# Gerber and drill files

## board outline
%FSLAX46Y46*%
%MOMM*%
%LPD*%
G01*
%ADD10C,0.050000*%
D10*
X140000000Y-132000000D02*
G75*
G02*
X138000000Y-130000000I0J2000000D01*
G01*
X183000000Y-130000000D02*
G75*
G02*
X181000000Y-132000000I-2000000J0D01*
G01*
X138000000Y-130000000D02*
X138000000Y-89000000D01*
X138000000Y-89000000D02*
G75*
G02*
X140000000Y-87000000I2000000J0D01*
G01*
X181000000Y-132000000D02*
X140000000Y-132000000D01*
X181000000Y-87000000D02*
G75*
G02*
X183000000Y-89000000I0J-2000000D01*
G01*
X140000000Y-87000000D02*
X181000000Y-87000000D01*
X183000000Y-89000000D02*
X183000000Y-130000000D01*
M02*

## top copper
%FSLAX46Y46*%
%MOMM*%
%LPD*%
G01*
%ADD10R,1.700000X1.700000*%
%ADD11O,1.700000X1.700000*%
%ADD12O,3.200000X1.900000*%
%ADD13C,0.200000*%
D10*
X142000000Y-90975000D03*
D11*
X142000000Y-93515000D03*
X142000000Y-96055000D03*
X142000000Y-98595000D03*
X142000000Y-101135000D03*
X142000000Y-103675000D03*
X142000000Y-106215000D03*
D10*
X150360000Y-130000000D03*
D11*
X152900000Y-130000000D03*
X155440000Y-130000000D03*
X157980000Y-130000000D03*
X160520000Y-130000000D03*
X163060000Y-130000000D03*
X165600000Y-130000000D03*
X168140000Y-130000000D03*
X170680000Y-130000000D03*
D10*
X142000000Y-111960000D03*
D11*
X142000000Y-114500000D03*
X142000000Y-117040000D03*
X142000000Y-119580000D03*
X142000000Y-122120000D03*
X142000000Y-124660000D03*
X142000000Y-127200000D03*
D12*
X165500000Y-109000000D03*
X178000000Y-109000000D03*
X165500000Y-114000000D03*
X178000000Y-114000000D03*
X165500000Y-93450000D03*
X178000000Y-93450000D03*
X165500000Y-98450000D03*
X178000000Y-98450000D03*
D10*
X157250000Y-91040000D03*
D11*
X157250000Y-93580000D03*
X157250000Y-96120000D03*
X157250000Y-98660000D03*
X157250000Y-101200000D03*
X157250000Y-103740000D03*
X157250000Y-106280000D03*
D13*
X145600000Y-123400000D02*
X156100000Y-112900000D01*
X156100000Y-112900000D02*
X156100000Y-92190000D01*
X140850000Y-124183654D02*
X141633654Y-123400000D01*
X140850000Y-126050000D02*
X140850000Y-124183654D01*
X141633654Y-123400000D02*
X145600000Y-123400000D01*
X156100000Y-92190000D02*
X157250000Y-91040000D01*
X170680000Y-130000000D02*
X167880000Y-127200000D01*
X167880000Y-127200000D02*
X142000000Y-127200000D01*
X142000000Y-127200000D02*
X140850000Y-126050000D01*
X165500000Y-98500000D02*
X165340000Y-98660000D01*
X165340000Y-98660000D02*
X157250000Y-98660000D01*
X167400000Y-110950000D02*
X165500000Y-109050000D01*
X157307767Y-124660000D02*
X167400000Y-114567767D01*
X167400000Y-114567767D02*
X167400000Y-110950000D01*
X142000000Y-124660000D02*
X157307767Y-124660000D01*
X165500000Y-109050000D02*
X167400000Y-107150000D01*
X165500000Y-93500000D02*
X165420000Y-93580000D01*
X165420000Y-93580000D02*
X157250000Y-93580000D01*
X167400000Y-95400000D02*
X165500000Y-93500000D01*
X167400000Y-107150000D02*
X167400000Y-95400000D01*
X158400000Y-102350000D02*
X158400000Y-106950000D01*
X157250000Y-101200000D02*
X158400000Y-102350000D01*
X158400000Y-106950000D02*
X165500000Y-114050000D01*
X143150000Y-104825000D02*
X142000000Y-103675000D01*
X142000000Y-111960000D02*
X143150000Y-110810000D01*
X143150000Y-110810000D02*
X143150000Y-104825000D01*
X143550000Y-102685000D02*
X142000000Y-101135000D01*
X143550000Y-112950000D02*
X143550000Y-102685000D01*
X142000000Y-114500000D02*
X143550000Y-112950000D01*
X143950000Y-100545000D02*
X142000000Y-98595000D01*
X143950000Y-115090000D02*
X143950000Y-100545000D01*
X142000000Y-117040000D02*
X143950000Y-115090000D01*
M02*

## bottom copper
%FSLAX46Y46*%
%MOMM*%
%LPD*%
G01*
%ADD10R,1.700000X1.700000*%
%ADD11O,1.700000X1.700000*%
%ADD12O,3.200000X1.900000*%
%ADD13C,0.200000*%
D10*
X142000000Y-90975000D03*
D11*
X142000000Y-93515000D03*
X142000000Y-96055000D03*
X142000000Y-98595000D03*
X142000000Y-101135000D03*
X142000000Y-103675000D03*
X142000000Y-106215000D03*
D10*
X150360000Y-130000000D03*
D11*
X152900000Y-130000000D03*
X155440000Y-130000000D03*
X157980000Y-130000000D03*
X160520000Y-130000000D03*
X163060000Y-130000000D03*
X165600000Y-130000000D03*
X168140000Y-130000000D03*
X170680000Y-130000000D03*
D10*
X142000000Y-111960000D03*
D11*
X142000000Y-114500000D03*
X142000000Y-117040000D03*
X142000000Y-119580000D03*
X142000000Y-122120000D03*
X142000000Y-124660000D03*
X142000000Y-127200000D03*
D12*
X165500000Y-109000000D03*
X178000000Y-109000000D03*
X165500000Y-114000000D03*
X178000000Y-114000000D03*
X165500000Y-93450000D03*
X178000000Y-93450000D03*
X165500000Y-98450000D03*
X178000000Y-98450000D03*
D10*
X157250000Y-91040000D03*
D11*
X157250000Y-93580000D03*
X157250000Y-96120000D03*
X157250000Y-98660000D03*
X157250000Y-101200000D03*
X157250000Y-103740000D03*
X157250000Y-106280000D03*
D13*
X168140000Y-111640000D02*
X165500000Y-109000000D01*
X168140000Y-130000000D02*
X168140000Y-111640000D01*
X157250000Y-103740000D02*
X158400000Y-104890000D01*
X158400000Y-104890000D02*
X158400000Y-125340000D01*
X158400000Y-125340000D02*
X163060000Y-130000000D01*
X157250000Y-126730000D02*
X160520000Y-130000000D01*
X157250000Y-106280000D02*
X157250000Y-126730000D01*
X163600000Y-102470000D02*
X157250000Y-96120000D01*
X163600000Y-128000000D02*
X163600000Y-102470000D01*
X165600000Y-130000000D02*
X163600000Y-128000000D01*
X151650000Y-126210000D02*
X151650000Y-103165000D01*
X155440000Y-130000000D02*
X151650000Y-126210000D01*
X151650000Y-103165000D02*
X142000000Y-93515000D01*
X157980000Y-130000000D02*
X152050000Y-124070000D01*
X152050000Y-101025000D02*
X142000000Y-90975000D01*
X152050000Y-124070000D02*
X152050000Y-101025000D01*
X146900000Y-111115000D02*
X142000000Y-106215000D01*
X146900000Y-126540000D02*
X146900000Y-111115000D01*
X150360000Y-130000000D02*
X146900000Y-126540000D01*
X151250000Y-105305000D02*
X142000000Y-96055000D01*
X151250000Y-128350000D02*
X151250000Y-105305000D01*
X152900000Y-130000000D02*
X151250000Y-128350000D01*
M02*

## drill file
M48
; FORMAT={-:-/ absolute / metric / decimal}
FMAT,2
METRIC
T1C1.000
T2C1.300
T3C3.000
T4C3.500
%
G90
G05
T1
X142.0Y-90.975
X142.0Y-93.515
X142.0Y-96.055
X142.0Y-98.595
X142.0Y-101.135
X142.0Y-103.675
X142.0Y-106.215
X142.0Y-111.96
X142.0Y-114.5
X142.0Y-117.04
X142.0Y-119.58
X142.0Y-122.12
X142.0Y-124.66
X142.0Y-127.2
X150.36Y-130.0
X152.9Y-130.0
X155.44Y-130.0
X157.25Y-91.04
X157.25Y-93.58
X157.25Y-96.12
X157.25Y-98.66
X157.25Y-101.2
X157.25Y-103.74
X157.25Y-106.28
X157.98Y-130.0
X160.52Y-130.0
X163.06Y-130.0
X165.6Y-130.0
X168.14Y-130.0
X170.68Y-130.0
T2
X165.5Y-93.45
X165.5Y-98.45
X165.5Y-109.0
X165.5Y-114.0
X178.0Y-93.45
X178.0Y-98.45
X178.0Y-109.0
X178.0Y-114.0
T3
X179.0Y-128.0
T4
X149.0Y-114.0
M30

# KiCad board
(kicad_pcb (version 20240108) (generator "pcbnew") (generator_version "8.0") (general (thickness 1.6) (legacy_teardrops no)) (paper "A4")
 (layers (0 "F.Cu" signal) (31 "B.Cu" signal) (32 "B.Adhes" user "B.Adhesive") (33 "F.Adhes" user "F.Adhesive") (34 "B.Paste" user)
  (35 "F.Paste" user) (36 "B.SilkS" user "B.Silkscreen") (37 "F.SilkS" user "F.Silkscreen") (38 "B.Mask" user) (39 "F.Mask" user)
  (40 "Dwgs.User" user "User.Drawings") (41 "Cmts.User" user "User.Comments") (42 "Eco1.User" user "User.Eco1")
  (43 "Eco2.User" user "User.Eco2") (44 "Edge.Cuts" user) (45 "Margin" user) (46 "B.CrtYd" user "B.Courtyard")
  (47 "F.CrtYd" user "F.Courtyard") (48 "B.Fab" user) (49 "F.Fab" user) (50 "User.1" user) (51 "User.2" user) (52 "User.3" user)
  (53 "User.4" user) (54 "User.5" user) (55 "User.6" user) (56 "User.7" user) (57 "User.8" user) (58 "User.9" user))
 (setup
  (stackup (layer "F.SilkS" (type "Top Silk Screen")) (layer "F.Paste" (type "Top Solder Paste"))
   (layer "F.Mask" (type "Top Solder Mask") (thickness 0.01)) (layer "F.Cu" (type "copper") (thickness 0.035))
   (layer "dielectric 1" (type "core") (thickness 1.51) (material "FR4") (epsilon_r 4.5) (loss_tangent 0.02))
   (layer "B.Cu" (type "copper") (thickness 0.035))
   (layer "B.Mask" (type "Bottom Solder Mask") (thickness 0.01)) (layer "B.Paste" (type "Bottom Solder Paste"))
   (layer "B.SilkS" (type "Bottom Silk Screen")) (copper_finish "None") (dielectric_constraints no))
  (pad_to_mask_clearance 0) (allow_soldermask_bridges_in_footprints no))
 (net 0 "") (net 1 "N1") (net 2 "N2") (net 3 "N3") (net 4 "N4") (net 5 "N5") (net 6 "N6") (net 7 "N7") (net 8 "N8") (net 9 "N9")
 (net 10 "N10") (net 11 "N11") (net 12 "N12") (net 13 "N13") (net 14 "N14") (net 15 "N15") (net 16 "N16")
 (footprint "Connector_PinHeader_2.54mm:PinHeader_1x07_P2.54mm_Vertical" (layer "F.Cu") (at 142 90.975)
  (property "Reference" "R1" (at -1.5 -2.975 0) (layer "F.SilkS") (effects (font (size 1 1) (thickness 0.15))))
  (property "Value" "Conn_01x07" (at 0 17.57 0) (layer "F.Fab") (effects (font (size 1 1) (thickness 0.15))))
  (pad "1" thru_hole rect (at 0 0) (size 1.7 1.7) (drill 1) (layers "*.Cu" "*.Mask") (remove_unused_layers no) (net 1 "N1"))
  (pad "2" thru_hole oval (at 0 2.54) (size 1.7 1.7) (drill 1) (layers "*.Cu" "*.Mask") (remove_unused_layers no) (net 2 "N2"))
  (pad "3" thru_hole oval (at 0 5.08) (size 1.7 1.7) (drill 1) (layers "*.Cu" "*.Mask") (remove_unused_layers no) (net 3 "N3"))
  (pad "4" thru_hole oval (at 0 7.62) (size 1.7 1.7) (drill 1) (layers "*.Cu" "*.Mask") (remove_unused_layers no) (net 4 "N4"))
  (pad "5" thru_hole oval (at 0 10.16) (size 1.7 1.7) (drill 1) (layers "*.Cu" "*.Mask") (remove_unused_layers no) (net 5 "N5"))
  (pad "6" thru_hole oval (at 0 12.7) (size 1.7 1.7) (drill 1) (layers "*.Cu" "*.Mask") (remove_unused_layers no) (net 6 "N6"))
  (pad "7" thru_hole oval (at 0 15.24) (size 1.7 1.7) (drill 1) (layers "*.Cu" "*.Mask") (remove_unused_layers no) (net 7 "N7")))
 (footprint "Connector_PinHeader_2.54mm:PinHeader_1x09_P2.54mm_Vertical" (layer "F.Cu") (at 150.36 130 90)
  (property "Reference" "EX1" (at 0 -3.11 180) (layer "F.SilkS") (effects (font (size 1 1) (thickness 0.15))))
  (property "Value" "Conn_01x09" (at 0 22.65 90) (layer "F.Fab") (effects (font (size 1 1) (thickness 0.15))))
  (pad "1" thru_hole rect (at 0 0 90) (size 1.7 1.7) (drill 1) (layers "*.Cu" "*.Mask") (remove_unused_layers no) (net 7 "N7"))
  (pad "2" thru_hole oval (at 0 2.54 90) (size 1.7 1.7) (drill 1) (layers "*.Cu" "*.Mask") (remove_unused_layers no) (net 3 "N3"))
  (pad "3" thru_hole oval (at 0 5.08 90) (size 1.7 1.7) (drill 1) (layers "*.Cu" "*.Mask") (remove_unused_layers no) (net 2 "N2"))
  (pad "4" thru_hole oval (at 0 7.62 90) (size 1.7 1.7) (drill 1) (layers "*.Cu" "*.Mask") (remove_unused_layers no) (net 1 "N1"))
  (pad "5" thru_hole oval (at 0 10.16 90) (size 1.7 1.7) (drill 1) (layers "*.Cu" "*.Mask") (remove_unused_layers no) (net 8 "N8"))
  (pad "6" thru_hole oval (at 0 12.7 90) (size 1.7 1.7) (drill 1) (layers "*.Cu" "*.Mask") (remove_unused_layers no) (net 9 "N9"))
  (pad "7" thru_hole oval (at 0 15.24 90) (size 1.7 1.7) (drill 1) (layers "*.Cu" "*.Mask") (remove_unused_layers no) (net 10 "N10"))
  (pad "8" thru_hole oval (at 0 17.78 90) (size 1.7 1.7) (drill 1) (layers "*.Cu" "*.Mask") (remove_unused_layers no) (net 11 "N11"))
  (pad "9" thru_hole oval (at 0 20.32 90) (size 1.7 1.7) (drill 1) (layers "*.Cu" "*.Mask") (remove_unused_layers no) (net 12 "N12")))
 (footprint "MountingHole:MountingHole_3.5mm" (layer "F.Cu") (at 149 114)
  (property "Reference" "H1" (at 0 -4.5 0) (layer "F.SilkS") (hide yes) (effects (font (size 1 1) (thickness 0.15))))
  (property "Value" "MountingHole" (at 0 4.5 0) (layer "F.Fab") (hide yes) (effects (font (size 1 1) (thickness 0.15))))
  (pad "" np_thru_hole circle (at 0 0) (size 3.5 3.5) (drill 3.5) (layers "*.Cu" "*.Mask")))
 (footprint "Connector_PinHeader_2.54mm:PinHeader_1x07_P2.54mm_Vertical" (layer "F.Cu") (at 142 111.96)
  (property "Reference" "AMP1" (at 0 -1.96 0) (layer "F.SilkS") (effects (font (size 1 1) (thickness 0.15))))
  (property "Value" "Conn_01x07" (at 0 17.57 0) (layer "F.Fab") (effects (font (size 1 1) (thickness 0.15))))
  (pad "1" thru_hole rect (at 0 0) (size 1.7 1.7) (drill 1) (layers "*.Cu" "*.Mask") (remove_unused_layers no) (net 6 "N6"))
  (pad "2" thru_hole oval (at 0 2.54) (size 1.7 1.7) (drill 1) (layers "*.Cu" "*.Mask") (remove_unused_layers no) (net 5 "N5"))
  (pad "3" thru_hole oval (at 0 5.08) (size 1.7 1.7) (drill 1) (layers "*.Cu" "*.Mask") (remove_unused_layers no) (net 4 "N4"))
  (pad "4" thru_hole oval (at 0 7.62) (size 1.7 1.7) (drill 1) (layers "*.Cu" "*.Mask") (remove_unused_layers no) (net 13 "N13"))
  (pad "5" thru_hole oval (at 0 10.16) (size 1.7 1.7) (drill 1) (layers "*.Cu" "*.Mask") (remove_unused_layers no) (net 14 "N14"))
  (pad "6" thru_hole oval (at 0 12.7) (size 1.7 1.7) (drill 1) (layers "*.Cu" "*.Mask") (remove_unused_layers no) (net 11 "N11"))
  (pad "7" thru_hole oval (at 0 15.24) (size 1.7 1.7) (drill 1) (layers "*.Cu" "*.Mask") (remove_unused_layers no) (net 12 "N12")))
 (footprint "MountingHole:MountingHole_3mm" (layer "F.Cu") (at 179 128)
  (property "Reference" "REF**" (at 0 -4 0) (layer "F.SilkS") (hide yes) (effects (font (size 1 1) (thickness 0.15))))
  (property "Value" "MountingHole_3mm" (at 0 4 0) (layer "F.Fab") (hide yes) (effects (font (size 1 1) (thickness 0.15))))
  (pad "" np_thru_hole circle (at 0 0) (size 3 3) (drill 3) (layers "*.Cu" "*.Mask")))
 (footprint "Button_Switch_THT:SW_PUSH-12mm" (layer "F.Cu") (at 165.5 109)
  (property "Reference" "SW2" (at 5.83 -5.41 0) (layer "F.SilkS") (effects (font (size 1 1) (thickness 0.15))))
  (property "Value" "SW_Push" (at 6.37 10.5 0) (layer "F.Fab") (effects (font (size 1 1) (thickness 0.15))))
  (pad "1" thru_hole oval (at 0 0) (size 3.2 1.9) (drill 1.3) (layers "*.Cu" "*.Mask") (remove_unused_layers no) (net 11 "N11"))
  (pad "1" thru_hole oval (at 12.5 0) (size 3.2 1.9) (drill 1.3) (layers "*.Cu" "*.Mask") (remove_unused_layers no))
  (pad "2" thru_hole oval (at 0 5) (size 3.2 1.9) (drill 1.3) (layers "*.Cu" "*.Mask") (remove_unused_layers no) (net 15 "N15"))
  (pad "2" thru_hole oval (at 12.5 5) (size 3.2 1.9) (drill 1.3) (layers "*.Cu" "*.Mask") (remove_unused_layers no)))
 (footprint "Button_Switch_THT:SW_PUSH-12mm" (layer "F.Cu") (at 165.5 93.45)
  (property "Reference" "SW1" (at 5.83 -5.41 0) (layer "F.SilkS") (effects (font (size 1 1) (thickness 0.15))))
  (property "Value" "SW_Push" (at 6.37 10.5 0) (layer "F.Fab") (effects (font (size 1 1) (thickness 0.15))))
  (pad "1" thru_hole oval (at 0 0) (size 3.2 1.9) (drill 1.3) (layers "*.Cu" "*.Mask") (remove_unused_layers no) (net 11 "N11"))
  (pad "1" thru_hole oval (at 12.5 0) (size 3.2 1.9) (drill 1.3) (layers "*.Cu" "*.Mask") (remove_unused_layers no))
  (pad "2" thru_hole oval (at 0 5) (size 3.2 1.9) (drill 1.3) (layers "*.Cu" "*.Mask") (remove_unused_layers no) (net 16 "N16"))
  (pad "2" thru_hole oval (at 12.5 5) (size 3.2 1.9) (drill 1.3) (layers "*.Cu" "*.Mask") (remove_unused_layers no)))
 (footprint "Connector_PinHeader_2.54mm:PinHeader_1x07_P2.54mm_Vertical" (layer "F.Cu") (at 157.25 91.04)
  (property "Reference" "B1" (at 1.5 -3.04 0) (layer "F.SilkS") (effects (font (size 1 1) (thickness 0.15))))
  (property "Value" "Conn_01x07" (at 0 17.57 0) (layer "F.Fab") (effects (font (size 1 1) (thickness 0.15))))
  (pad "1" thru_hole rect (at 0 0) (size 1.7 1.7) (drill 1) (layers "*.Cu" "*.Mask") (remove_unused_layers no) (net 12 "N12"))
  (pad "2" thru_hole oval (at 0 2.54) (size 1.7 1.7) (drill 1) (layers "*.Cu" "*.Mask") (remove_unused_layers no) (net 11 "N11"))
  (pad "3" thru_hole oval (at 0 5.08) (size 1.7 1.7) (drill 1) (layers "*.Cu" "*.Mask") (remove_unused_layers no) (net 10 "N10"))
  (pad "4" thru_hole oval (at 0 7.62) (size 1.7 1.7) (drill 1) (layers "*.Cu" "*.Mask") (remove_unused_layers no) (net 16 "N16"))
  (pad "5" thru_hole oval (at 0 10.16) (size 1.7 1.7) (drill 1) (layers "*.Cu" "*.Mask") (remove_unused_layers no) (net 15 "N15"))
  (pad "6" thru_hole oval (at 0 12.7) (size 1.7 1.7) (drill 1) (layers "*.Cu" "*.Mask") (remove_unused_layers no) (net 9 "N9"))
  (pad "7" thru_hole oval (at 0 15.24) (size 1.7 1.7) (drill 1) (layers "*.Cu" "*.Mask") (remove_unused_layers no) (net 8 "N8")))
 (gr_arc (start 140 132) (mid 138.585786 131.414214) (end 138 130) (stroke (width 0.05) (type default)) (layer "Edge.Cuts"))
 (gr_arc (start 183 130) (mid 182.414214 131.414214) (end 181 132) (stroke (width 0.05) (type default)) (layer "Edge.Cuts"))
 (gr_line (start 138 130) (end 138 89) (stroke (width 0.05) (type default)) (layer "Edge.Cuts"))
 (gr_arc (start 138 89) (mid 138.585786 87.585786) (end 140 87) (stroke (width 0.05) (type default)) (layer "Edge.Cuts"))
 (gr_line (start 181 132) (end 140 132) (stroke (width 0.05) (type default)) (layer "Edge.Cuts"))
 (gr_arc (start 181 87) (mid 182.414214 87.585786) (end 183 89) (stroke (width 0.05) (type default)) (layer "Edge.Cuts"))
 (gr_line (start 140 87) (end 181 87) (stroke (width 0.05) (type default)) (layer "Edge.Cuts"))
 (gr_line (start 183 89) (end 183 130) (stroke (width 0.05) (type default)) (layer "Edge.Cuts"))
 (segment (start 145.6 123.4) (end 156.1 112.9) (width 0.2) (layer "F.Cu") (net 12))
 (segment (start 156.1 112.9) (end 156.1 92.19) (width 0.2) (layer "F.Cu") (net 12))
 (segment (start 140.85 124.183654) (end 141.633654 123.4) (width 0.2) (layer "F.Cu") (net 12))
 (segment (start 140.85 126.05) (end 140.85 124.183654) (width 0.2) (layer "F.Cu") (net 12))
 (segment (start 141.633654 123.4) (end 145.6 123.4) (width 0.2) (layer "F.Cu") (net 12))
 (segment (start 156.1 92.19) (end 157.25 91.04) (width 0.2) (layer "F.Cu") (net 12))
 (segment (start 170.68 130) (end 167.88 127.2) (width 0.2) (layer "F.Cu") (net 12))
 (segment (start 167.88 127.2) (end 142 127.2) (width 0.2) (layer "F.Cu") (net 12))
 (segment (start 142 127.2) (end 140.85 126.05) (width 0.2) (layer "F.Cu") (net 12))
 (segment (start 165.5 98.5) (end 165.34 98.66) (width 0.2) (layer "F.Cu") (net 16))
 (segment (start 165.34 98.66) (end 157.25 98.66) (width 0.2) (layer "F.Cu") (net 16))
 (segment (start 167.4 110.95) (end 165.5 109.05) (width 0.2) (layer "F.Cu") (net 11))
 (segment (start 157.307767 124.66) (end 167.4 114.567767) (width 0.2) (layer "F.Cu") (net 11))
 (segment (start 167.4 114.567767) (end 167.4 110.95) (width 0.2) (layer "F.Cu") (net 11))
 (segment (start 142 124.66) (end 157.307767 124.66) (width 0.2) (layer "F.Cu") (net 11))
 (segment (start 165.5 109.05) (end 167.4 107.15) (width 0.2) (layer "F.Cu") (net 11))
 (segment (start 165.5 93.5) (end 165.42 93.58) (width 0.2) (layer "F.Cu") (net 11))
 (segment (start 165.42 93.58) (end 157.25 93.58) (width 0.2) (layer "F.Cu") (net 11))
 (segment (start 167.4 95.4) (end 165.5 93.5) (width 0.2) (layer "F.Cu") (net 11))
 (segment (start 167.4 107.15) (end 167.4 95.4) (width 0.2) (layer "F.Cu") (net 11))
 (segment (start 168.14 111.64) (end 165.5 109) (width 0.2) (layer "B.Cu") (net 11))
 (segment (start 168.14 130) (end 168.14 111.64) (width 0.2) (layer "B.Cu") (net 11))
 (segment (start 158.4 102.35) (end 158.4 106.95) (width 0.2) (layer "F.Cu") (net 15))
 (segment (start 157.25 101.2) (end 158.4 102.35) (width 0.2) (layer "F.Cu") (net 15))
 (segment (start 158.4 106.95) (end 165.5 114.05) (width 0.2) (layer "F.Cu") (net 15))
 (segment (start 143.15 104.825) (end 142 103.675) (width 0.2) (layer "F.Cu") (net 6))
 (segment (start 142 111.96) (end 143.15 110.81) (width 0.2) (layer "F.Cu") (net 6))
 (segment (start 143.15 110.81) (end 143.15 104.825) (width 0.2) (layer "F.Cu") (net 6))
 (segment (start 143.55 102.685) (end 142 101.135) (width 0.2) (layer "F.Cu") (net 5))
 (segment (start 143.55 112.95) (end 143.55 102.685) (width 0.2) (layer "F.Cu") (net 5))
 (segment (start 142 114.5) (end 143.55 112.95) (width 0.2) (layer "F.Cu") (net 5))
 (segment (start 143.95 100.545) (end 142 98.595) (width 0.2) (layer "F.Cu") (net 4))
 (segment (start 143.95 115.09) (end 143.95 100.545) (width 0.2) (layer "F.Cu") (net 4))
 (segment (start 142 117.04) (end 143.95 115.09) (width 0.2) (layer "F.Cu") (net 4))
 (segment (start 157.25 103.74) (end 158.4 104.89) (width 0.2) (layer "B.Cu") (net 9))
 (segment (start 158.4 104.89) (end 158.4 125.34) (width 0.2) (layer "B.Cu") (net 9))
 (segment (start 158.4 125.34) (end 163.06 130) (width 0.2) (layer "B.Cu") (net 9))
 (segment (start 157.25 126.73) (end 160.52 130) (width 0.2) (layer "B.Cu") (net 8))
 (segment (start 157.25 106.28) (end 157.25 126.73) (width 0.2) (layer "B.Cu") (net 8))
 (segment (start 163.6 102.47) (end 157.25 96.12) (width 0.2) (layer "B.Cu") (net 10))
 (segment (start 163.6 128) (end 163.6 102.47) (width 0.2) (layer "B.Cu") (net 10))
 (segment (start 165.6 130) (end 163.6 128) (width 0.2) (layer "B.Cu") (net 10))
 (segment (start 151.65 126.21) (end 151.65 103.165) (width 0.2) (layer "B.Cu") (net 2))
 (segment (start 155.44 130) (end 151.65 126.21) (width 0.2) (layer "B.Cu") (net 2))
 (segment (start 151.65 103.165) (end 142 93.515) (width 0.2) (layer "B.Cu") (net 2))
 (segment (start 157.98 130) (end 152.05 124.07) (width 0.2) (layer "B.Cu") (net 1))
 (segment (start 152.05 101.025) (end 142 90.975) (width 0.2) (layer "B.Cu") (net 1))
 (segment (start 152.05 124.07) (end 152.05 101.025) (width 0.2) (layer "B.Cu") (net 1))
 (segment (start 146.9 111.115) (end 142 106.215) (width 0.2) (layer "B.Cu") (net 7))
 (segment (start 146.9 126.54) (end 146.9 111.115) (width 0.2) (layer "B.Cu") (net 7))
 (segment (start 150.36 130) (end 146.9 126.54) (width 0.2) (layer "B.Cu") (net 7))
 (segment (start 151.25 105.305) (end 142 96.055) (width 0.2) (layer "B.Cu") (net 3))
 (segment (start 151.25 128.35) (end 151.25 105.305) (width 0.2) (layer "B.Cu") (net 3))
 (segment (start 152.9 130) (end 151.25 128.35) (width 0.2) (layer "B.Cu") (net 3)))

